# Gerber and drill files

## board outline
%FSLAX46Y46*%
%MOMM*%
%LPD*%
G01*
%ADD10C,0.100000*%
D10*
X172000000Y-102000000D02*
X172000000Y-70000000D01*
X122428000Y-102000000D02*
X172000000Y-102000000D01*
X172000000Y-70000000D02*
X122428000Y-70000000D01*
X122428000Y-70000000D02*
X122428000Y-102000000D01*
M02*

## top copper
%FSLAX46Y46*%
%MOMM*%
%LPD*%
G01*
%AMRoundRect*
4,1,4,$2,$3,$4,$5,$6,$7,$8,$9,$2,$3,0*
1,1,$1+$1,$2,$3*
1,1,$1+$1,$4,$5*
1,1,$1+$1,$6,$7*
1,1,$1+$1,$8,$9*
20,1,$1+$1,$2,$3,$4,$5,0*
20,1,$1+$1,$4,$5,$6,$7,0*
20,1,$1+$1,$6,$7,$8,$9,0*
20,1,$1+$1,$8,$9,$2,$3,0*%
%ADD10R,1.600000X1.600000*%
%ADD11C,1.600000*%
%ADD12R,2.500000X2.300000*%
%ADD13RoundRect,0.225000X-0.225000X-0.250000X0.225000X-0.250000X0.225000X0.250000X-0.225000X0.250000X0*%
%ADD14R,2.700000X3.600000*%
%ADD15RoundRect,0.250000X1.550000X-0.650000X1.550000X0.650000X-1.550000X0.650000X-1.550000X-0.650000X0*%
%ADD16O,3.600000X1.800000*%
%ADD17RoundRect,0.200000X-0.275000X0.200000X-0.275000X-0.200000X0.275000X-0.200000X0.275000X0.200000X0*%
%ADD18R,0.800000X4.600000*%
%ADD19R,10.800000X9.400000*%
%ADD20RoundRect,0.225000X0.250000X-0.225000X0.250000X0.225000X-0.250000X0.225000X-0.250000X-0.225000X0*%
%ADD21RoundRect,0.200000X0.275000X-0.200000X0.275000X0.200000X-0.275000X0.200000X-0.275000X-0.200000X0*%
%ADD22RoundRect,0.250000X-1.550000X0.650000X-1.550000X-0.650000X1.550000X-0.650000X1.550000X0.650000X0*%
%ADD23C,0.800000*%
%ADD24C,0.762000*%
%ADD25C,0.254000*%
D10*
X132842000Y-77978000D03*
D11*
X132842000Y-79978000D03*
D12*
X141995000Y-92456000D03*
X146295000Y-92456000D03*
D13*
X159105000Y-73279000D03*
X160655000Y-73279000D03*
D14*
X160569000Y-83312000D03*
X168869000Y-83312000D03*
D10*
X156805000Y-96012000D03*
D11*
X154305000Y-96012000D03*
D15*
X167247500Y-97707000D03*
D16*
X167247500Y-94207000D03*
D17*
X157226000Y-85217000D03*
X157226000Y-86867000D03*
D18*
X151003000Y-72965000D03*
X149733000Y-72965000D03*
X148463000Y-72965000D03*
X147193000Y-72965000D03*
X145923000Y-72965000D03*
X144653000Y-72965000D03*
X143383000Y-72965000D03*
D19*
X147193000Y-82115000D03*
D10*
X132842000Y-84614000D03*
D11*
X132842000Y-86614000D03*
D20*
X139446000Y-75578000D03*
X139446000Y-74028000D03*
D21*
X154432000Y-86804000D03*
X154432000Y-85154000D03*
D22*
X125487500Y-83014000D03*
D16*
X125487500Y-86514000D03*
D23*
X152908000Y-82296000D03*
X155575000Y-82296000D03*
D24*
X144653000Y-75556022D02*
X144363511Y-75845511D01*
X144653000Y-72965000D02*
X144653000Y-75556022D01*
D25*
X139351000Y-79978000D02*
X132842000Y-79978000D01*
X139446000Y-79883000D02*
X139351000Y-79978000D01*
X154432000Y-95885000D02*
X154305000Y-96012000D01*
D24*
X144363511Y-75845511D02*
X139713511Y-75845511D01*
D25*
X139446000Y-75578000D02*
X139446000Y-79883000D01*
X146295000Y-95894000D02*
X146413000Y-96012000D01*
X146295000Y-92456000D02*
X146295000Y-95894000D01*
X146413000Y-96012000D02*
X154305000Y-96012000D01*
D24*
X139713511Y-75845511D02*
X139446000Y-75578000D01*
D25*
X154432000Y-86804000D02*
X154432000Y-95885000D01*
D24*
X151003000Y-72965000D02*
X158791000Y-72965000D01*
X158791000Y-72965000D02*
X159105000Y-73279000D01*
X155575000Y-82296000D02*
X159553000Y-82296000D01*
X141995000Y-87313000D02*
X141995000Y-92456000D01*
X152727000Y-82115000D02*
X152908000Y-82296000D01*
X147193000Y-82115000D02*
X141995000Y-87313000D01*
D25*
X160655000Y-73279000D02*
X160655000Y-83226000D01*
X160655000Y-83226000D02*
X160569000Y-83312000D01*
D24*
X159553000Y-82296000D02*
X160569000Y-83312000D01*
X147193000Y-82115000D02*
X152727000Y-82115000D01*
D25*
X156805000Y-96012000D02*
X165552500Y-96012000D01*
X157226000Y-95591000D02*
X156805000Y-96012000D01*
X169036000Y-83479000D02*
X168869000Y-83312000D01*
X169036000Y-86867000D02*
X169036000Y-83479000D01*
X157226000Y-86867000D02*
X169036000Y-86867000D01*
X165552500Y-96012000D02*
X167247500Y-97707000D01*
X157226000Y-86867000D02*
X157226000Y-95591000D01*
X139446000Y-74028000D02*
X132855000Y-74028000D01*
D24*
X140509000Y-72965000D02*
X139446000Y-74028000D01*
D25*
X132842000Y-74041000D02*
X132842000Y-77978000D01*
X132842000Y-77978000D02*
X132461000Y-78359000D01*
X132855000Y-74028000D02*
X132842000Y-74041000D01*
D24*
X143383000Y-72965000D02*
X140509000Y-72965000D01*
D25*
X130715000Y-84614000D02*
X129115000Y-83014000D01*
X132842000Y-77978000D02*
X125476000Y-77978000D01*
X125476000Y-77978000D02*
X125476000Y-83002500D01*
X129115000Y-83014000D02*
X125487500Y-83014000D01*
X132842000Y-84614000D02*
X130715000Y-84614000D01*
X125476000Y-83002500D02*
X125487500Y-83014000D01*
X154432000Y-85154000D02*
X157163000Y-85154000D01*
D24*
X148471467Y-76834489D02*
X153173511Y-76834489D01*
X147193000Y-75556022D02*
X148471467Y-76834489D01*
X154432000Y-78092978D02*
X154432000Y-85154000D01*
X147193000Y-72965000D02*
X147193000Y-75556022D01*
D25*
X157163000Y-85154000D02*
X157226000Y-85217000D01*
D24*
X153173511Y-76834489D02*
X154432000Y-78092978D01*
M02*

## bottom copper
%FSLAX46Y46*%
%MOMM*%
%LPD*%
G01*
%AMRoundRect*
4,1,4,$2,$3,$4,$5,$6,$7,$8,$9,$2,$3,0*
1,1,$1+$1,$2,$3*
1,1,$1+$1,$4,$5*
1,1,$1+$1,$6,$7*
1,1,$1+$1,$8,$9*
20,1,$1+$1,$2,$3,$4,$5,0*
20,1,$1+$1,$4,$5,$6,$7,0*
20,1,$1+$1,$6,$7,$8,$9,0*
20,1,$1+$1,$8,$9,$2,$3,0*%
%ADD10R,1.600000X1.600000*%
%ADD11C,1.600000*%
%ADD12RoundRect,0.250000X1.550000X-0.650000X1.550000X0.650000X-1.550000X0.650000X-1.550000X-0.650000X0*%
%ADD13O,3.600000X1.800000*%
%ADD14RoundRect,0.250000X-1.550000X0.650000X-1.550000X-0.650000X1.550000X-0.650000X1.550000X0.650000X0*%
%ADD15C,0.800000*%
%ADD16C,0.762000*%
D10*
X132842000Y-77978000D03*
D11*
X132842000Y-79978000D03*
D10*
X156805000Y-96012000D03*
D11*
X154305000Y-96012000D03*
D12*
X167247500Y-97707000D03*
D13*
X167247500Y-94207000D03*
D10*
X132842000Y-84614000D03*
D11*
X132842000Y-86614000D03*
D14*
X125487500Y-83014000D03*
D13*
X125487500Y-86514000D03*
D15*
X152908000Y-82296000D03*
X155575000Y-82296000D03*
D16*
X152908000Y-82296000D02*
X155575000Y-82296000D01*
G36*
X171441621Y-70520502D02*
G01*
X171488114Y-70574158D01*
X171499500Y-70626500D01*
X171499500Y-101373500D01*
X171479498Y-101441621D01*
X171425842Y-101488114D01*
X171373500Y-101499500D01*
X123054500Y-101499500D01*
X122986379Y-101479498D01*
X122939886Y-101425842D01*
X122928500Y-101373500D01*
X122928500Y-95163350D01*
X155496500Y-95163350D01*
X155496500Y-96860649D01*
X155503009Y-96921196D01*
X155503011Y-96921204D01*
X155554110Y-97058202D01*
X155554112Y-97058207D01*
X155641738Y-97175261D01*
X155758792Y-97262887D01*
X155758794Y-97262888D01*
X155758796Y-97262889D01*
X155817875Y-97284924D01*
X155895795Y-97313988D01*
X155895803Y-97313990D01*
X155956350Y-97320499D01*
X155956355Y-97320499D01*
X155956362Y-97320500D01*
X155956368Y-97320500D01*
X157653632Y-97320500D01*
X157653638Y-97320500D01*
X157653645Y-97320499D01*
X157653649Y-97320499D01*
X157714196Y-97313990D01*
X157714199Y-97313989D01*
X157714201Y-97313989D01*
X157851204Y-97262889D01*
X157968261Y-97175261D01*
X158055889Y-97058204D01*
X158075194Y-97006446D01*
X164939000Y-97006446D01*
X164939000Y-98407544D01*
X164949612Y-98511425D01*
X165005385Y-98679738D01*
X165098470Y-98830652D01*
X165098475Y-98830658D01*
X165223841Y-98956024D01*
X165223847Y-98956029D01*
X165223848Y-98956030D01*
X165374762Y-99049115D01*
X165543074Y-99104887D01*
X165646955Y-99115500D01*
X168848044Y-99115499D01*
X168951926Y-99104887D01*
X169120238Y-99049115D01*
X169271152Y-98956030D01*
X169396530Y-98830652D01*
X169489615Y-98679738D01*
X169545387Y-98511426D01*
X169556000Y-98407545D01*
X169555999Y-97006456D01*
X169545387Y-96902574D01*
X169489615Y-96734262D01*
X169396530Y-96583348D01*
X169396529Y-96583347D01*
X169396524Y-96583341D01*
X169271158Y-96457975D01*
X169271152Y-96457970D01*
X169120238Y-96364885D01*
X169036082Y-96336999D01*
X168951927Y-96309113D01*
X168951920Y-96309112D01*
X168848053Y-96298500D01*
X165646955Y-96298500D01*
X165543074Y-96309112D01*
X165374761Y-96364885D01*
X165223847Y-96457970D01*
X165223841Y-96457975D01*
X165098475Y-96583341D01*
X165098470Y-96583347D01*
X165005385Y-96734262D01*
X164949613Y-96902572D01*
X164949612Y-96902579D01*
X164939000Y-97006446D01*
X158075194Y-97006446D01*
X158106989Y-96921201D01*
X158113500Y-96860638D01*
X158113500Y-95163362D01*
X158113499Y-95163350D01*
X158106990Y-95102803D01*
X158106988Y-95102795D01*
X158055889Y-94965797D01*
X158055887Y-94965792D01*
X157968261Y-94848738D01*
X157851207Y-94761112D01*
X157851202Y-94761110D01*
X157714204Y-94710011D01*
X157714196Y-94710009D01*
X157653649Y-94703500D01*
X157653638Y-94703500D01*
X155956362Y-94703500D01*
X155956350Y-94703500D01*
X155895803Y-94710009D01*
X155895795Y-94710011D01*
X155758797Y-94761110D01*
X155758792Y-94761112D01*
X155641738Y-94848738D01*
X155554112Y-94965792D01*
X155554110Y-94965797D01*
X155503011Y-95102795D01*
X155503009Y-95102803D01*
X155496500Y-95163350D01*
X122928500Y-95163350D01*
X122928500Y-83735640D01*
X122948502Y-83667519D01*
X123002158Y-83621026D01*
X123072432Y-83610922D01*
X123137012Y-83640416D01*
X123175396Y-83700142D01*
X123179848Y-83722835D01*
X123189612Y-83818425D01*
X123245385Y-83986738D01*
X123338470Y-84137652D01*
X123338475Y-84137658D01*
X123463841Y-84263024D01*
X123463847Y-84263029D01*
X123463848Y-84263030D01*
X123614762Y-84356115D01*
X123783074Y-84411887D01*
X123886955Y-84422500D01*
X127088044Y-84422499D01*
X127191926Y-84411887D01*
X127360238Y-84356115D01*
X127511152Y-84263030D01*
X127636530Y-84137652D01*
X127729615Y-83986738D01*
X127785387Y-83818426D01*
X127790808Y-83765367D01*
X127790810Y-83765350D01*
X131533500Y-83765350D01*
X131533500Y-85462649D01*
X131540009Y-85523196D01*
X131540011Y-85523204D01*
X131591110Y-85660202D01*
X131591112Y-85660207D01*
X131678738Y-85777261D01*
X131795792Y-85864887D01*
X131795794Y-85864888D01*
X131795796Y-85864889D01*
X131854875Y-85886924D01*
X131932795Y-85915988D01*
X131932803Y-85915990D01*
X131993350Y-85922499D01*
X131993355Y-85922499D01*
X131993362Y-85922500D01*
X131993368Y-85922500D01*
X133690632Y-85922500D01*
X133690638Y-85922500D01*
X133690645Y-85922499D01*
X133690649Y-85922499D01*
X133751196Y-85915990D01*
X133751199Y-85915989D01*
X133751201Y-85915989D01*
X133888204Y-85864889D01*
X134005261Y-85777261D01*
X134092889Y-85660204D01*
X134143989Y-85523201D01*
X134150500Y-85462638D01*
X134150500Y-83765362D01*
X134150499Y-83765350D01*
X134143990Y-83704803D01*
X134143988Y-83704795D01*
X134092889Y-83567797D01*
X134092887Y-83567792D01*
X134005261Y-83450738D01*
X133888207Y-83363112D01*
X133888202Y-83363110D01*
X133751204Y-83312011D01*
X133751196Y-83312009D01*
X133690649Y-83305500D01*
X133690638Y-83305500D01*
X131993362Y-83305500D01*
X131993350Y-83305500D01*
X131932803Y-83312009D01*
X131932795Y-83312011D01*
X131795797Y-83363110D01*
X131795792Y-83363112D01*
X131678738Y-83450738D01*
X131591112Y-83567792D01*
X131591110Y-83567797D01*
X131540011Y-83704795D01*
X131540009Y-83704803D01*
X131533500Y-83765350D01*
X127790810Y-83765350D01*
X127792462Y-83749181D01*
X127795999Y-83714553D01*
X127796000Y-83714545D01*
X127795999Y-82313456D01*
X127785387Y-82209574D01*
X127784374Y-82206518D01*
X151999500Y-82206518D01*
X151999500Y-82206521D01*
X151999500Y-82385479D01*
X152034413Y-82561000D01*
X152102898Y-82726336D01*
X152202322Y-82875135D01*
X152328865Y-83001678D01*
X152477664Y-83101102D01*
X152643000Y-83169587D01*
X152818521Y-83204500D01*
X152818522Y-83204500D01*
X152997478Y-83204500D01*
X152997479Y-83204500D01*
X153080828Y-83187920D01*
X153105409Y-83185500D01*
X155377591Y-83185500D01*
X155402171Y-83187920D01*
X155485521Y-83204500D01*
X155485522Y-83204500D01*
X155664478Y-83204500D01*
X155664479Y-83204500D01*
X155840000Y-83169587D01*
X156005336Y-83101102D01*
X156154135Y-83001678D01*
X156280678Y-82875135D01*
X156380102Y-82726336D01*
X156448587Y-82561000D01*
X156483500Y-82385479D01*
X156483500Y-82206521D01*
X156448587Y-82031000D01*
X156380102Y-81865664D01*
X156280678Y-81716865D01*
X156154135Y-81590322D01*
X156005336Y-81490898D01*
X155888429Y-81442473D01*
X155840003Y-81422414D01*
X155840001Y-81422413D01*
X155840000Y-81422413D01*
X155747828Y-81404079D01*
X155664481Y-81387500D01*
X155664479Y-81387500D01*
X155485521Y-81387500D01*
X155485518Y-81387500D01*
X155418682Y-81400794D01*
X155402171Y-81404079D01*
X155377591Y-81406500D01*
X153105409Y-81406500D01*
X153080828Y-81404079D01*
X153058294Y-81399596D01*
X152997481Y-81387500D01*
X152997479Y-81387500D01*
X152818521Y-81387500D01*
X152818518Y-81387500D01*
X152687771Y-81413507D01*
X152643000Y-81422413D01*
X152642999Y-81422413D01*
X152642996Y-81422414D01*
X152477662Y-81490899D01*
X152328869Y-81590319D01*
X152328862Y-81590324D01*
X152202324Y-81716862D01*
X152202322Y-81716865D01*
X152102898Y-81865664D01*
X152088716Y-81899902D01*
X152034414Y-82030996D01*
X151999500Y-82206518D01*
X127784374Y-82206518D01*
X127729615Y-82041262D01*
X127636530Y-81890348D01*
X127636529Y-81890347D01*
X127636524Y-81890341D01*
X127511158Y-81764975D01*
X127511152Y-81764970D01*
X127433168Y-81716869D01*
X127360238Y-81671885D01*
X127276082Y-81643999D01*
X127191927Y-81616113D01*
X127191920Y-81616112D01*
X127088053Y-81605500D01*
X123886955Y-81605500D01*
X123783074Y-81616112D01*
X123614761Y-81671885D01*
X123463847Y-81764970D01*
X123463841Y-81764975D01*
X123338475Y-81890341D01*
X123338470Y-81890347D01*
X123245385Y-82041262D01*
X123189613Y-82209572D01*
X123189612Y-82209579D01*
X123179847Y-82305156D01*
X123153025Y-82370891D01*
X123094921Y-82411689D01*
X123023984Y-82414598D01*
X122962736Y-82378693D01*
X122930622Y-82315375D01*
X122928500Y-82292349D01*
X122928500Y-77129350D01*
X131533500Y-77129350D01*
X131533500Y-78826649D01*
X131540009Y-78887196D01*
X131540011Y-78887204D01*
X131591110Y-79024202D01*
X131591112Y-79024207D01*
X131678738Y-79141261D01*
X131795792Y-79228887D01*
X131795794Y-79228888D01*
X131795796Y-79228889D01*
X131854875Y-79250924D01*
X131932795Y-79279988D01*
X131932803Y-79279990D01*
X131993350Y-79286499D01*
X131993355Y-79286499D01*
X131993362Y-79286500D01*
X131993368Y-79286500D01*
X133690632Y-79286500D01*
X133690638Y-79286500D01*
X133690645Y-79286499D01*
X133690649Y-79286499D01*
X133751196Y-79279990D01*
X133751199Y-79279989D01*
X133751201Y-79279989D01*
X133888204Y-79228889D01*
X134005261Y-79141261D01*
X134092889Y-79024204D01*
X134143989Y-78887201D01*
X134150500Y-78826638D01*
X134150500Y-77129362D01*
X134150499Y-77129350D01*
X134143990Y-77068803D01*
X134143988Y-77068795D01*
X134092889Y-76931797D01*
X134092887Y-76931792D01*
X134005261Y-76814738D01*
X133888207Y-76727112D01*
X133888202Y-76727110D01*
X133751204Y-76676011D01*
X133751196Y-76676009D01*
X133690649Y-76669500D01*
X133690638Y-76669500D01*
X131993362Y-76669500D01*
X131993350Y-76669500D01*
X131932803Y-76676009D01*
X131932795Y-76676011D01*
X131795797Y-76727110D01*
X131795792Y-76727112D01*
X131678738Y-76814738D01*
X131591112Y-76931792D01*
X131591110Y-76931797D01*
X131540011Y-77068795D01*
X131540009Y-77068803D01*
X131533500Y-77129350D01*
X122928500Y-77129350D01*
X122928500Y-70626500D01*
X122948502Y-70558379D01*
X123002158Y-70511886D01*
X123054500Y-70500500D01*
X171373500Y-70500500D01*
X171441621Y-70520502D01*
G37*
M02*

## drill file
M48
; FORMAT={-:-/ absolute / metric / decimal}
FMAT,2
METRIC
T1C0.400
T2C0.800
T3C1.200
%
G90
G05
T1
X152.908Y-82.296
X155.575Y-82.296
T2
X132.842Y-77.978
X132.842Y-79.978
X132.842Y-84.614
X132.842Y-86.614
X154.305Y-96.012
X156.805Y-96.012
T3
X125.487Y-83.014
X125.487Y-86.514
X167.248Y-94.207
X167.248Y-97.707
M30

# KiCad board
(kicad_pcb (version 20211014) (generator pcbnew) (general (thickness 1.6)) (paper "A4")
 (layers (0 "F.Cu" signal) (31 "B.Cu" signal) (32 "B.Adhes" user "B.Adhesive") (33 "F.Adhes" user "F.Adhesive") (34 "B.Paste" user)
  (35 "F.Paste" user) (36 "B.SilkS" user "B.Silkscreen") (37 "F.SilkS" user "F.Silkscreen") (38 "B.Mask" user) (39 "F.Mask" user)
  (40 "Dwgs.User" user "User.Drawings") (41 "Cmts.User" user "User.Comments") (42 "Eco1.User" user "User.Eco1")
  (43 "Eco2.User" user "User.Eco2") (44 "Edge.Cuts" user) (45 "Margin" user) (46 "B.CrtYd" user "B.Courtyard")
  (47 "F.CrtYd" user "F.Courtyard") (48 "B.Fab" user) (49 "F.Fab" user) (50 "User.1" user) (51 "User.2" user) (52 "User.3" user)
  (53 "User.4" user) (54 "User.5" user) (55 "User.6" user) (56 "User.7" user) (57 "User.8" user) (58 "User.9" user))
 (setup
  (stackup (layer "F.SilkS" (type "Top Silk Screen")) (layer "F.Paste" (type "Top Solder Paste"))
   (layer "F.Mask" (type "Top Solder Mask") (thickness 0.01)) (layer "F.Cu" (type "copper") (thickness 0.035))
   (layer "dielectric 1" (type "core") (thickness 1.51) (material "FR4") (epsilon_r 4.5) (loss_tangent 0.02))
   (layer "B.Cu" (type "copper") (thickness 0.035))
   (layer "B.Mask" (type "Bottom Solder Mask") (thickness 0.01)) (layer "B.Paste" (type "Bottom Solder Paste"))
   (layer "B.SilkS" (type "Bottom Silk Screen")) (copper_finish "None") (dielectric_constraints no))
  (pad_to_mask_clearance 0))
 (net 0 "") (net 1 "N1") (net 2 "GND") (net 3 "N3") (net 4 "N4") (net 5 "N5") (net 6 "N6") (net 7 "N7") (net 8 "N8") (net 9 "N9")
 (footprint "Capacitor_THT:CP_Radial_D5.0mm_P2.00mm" (layer "F.Cu") (at 132.842 77.978 -90)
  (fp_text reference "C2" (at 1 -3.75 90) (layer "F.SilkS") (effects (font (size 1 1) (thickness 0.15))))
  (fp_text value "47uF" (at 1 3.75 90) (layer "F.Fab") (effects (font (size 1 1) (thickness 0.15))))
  (pad "1" thru_hole rect (at 0 0 270) (size 1.6 1.6) (drill 0.8) (layers *.Cu *.Mask) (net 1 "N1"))
  (pad "2" thru_hole circle (at 2 0 270) (size 1.6 1.6) (drill 0.8) (layers *.Cu *.Mask) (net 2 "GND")))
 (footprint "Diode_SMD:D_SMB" (layer "F.Cu") (at 144.145 92.456)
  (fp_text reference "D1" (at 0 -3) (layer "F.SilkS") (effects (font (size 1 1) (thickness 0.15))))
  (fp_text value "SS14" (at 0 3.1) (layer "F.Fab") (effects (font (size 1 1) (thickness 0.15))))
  (pad "1" smd rect (at -2.15 0) (size 2.5 2.3) (layers "F.Cu" "F.Paste" "F.Mask") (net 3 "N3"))
  (pad "2" smd rect (at 2.15 0) (size 2.5 2.3) (layers "F.Cu" "F.Paste" "F.Mask") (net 2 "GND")))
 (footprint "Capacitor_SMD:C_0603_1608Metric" (layer "F.Cu") (at 159.88 73.279)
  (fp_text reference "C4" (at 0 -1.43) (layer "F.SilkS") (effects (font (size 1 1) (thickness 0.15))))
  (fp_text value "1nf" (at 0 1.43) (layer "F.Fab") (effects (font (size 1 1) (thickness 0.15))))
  (pad "1" smd roundrect (at -0.775 0) (size 0.9 0.95) (layers "F.Cu" "F.Paste" "F.Mask") (roundrect_rratio 0.25) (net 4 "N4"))
  (pad "2" smd roundrect (at 0.775 0) (size 0.9 0.95) (layers "F.Cu" "F.Paste" "F.Mask") (roundrect_rratio 0.25) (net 3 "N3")))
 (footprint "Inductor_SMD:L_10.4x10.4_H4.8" (layer "F.Cu") (at 164.719 83.312)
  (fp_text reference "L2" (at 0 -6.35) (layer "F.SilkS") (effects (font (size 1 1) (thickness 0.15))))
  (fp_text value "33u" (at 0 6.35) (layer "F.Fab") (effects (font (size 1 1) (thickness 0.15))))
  (pad "1" smd rect (at -4.15 0) (size 2.7 3.6) (layers "F.Cu" "F.Paste" "F.Mask") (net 3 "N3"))
  (pad "2" smd rect (at 4.15 0) (size 2.7 3.6) (layers "F.Cu" "F.Paste" "F.Mask") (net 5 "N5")))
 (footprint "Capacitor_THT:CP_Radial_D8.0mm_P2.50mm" (layer "F.Cu") (at 156.805 96.012 180)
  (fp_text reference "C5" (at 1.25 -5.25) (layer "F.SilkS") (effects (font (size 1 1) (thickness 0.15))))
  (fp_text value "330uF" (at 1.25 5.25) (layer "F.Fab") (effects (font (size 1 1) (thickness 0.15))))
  (pad "1" thru_hole rect (at 0 0 180) (size 1.6 1.6) (drill 0.8) (layers *.Cu *.Mask) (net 5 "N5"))
  (pad "2" thru_hole circle (at 2.5 0 180) (size 1.6 1.6) (drill 0.8) (layers *.Cu *.Mask) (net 2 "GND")))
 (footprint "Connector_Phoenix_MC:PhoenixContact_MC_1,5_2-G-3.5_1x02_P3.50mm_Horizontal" (layer "F.Cu") (at 167.2475 97.707 90)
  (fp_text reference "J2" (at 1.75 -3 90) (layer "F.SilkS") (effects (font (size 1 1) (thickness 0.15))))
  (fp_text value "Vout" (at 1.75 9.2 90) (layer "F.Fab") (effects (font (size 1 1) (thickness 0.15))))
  (pad "1" thru_hole roundrect (at 0 0 90) (size 1.8 3.6) (drill 1.2) (layers *.Cu *.Mask) (roundrect_rratio 0.1388888889) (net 5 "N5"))
  (pad "2" thru_hole oval (at 3.5 0 90) (size 1.8 3.6) (drill 1.2) (layers *.Cu *.Mask) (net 2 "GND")))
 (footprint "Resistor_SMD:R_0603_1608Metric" (layer "F.Cu") (at 157.226 86.042 -90)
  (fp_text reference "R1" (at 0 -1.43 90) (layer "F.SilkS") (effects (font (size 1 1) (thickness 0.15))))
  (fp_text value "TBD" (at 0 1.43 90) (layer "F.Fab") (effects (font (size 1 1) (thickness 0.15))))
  (pad "1" smd roundrect (at -0.825 0 270) (size 0.8 0.95) (layers "F.Cu" "F.Paste" "F.Mask") (roundrect_rratio 0.25) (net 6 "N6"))
  (pad "2" smd roundrect (at 0.825 0 270) (size 0.8 0.95) (layers "F.Cu" "F.Paste" "F.Mask") (roundrect_rratio 0.25) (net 5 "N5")))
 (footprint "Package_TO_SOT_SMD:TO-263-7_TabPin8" (layer "F.Cu") (at 147.193 78.74 -90)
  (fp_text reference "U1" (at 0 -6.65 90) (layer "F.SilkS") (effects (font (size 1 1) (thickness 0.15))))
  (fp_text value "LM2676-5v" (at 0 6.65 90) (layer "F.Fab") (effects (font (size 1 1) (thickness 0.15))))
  (pad "" smd rect (at 0.95 2.775 270) (size 4.55 5.25) (layers "F.Paste"))
  (pad "" smd rect (at 5.8 -2.775 270) (size 4.55 5.25) (layers "F.Paste"))
  (pad "" smd rect (at 5.8 2.775 270) (size 4.55 5.25) (layers "F.Paste"))
  (pad "" smd rect (at 0.95 -2.775 270) (size 4.55 5.25) (layers "F.Paste"))
  (pad "1" smd rect (at -5.775 -3.81 270) (size 4.6 0.8) (layers "F.Cu" "F.Paste" "F.Mask") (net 4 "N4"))
  (pad "2" smd rect (at -5.775 -2.54 270) (size 4.6 0.8) (layers "F.Cu" "F.Paste" "F.Mask") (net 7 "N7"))
  (pad "3" smd rect (at -5.775 -1.27 270) (size 4.6 0.8) (layers "F.Cu" "F.Paste" "F.Mask") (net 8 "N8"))
  (pad "4" smd rect (at -5.775 0 270) (size 4.6 0.8) (layers "F.Cu" "F.Paste" "F.Mask") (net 6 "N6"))
  (pad "5" smd rect (at -5.775 1.27 270) (size 4.6 0.8) (layers "F.Cu" "F.Paste" "F.Mask") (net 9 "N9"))
  (pad "6" smd rect (at -5.775 2.54 270) (size 4.6 0.8) (layers "F.Cu" "F.Paste" "F.Mask") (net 2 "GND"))
  (pad "7" smd rect (at -5.775 3.81 270) (size 4.6 0.8) (layers "F.Cu" "F.Paste" "F.Mask") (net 1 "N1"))
  (pad "8" smd rect (at 3.375 0 270) (size 9.4 10.8) (layers "F.Cu" "F.Mask") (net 3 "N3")))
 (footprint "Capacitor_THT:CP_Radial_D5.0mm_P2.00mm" (layer "F.Cu") (at 132.842 84.614 -90)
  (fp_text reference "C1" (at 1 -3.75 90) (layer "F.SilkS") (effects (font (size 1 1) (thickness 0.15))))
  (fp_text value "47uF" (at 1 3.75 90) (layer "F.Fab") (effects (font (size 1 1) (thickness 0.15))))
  (pad "1" thru_hole rect (at 0 0 270) (size 1.6 1.6) (drill 0.8) (layers *.Cu *.Mask) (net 1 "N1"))
  (pad "2" thru_hole circle (at 2 0 270) (size 1.6 1.6) (drill 0.8) (layers *.Cu *.Mask) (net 2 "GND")))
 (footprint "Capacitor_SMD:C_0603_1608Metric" (layer "F.Cu") (at 139.446 74.803 90)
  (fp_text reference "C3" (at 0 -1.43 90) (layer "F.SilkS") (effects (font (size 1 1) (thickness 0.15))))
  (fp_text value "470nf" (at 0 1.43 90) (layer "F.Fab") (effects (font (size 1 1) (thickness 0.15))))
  (pad "1" smd roundrect (at -0.775 0 90) (size 0.9 0.95) (layers "F.Cu" "F.Paste" "F.Mask") (roundrect_rratio 0.25) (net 2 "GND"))
  (pad "2" smd roundrect (at 0.775 0 90) (size 0.9 0.95) (layers "F.Cu" "F.Paste" "F.Mask") (roundrect_rratio 0.25) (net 1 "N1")))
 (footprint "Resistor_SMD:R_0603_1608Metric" (layer "F.Cu") (at 154.432 85.979 90)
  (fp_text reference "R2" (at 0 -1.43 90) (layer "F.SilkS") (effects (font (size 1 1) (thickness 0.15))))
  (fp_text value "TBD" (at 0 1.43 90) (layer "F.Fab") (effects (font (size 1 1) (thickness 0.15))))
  (pad "1" smd roundrect (at -0.825 0 90) (size 0.8 0.95) (layers "F.Cu" "F.Paste" "F.Mask") (roundrect_rratio 0.25) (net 2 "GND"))
  (pad "2" smd roundrect (at 0.825 0 90) (size 0.8 0.95) (layers "F.Cu" "F.Paste" "F.Mask") (roundrect_rratio 0.25) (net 6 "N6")))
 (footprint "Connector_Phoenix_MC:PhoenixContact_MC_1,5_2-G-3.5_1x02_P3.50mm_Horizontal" (layer "F.Cu") (at 125.4875 83.014 -90)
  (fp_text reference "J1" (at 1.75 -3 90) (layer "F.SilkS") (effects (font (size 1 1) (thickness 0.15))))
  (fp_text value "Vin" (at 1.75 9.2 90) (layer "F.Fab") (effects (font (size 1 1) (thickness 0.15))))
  (pad "1" thru_hole roundrect (at 0 0 270) (size 1.8 3.6) (drill 1.2) (layers *.Cu *.Mask) (roundrect_rratio 0.1388888889) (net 1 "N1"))
  (pad "2" thru_hole oval (at 3.5 0 270) (size 1.8 3.6) (drill 1.2) (layers *.Cu *.Mask) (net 2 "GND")))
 (gr_line (start 172 102) (end 172 70) (layer "Edge.Cuts") (width 0.1))
 (gr_line (start 122.428 102) (end 172 102) (layer "Edge.Cuts") (width 0.1))
 (gr_line (start 172 70) (end 122.428 70) (layer "Edge.Cuts") (width 0.1))
 (gr_line (start 122.428 70) (end 122.428 102) (layer "Edge.Cuts") (width 0.1))
 (segment (start 144.653 75.556022) (end 144.363511 75.845511) (width 0.762) (layer "F.Cu") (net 2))
 (segment (start 144.653 72.965) (end 144.653 75.556022) (width 0.762) (layer "F.Cu") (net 2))
 (segment (start 139.351 79.978) (end 132.842 79.978) (width 0.254) (layer "F.Cu") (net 2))
 (segment (start 139.446 79.883) (end 139.351 79.978) (width 0.254) (layer "F.Cu") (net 2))
 (segment (start 154.432 95.885) (end 154.305 96.012) (width 0.254) (layer "F.Cu") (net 2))
 (segment (start 144.363511 75.845511) (end 139.713511 75.845511) (width 0.762) (layer "F.Cu") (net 2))
 (segment (start 139.446 75.578) (end 139.446 79.883) (width 0.254) (layer "F.Cu") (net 2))
 (segment (start 146.295 95.894) (end 146.413 96.012) (width 0.254) (layer "F.Cu") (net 2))
 (segment (start 146.295 92.456) (end 146.295 95.894) (width 0.254) (layer "F.Cu") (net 2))
 (segment (start 146.413 96.012) (end 154.305 96.012) (width 0.254) (layer "F.Cu") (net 2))
 (segment (start 139.713511 75.845511) (end 139.446 75.578) (width 0.762) (layer "F.Cu") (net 2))
 (segment (start 154.432 86.804) (end 154.432 95.885) (width 0.254) (layer "F.Cu") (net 2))
 (segment (start 151.003 72.965) (end 158.791 72.965) (width 0.762) (layer "F.Cu") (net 4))
 (segment (start 158.791 72.965) (end 159.105 73.279) (width 0.762) (layer "F.Cu") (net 4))
 (segment (start 155.575 82.296) (end 159.553 82.296) (width 0.762) (layer "F.Cu") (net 3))
 (segment (start 141.995 87.313) (end 141.995 92.456) (width 0.762) (layer "F.Cu") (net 3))
 (segment (start 152.727 82.115) (end 152.908 82.296) (width 0.762) (layer "F.Cu") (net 3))
 (segment (start 147.193 82.115) (end 141.995 87.313) (width 0.762) (layer "F.Cu") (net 3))
 (segment (start 160.655 73.279) (end 160.655 83.226) (width 0.254) (layer "F.Cu") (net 3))
 (segment (start 160.655 83.226) (end 160.569 83.312) (width 0.254) (layer "F.Cu") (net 3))
 (segment (start 159.553 82.296) (end 160.569 83.312) (width 0.762) (layer "F.Cu") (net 3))
 (segment (start 147.193 82.115) (end 152.727 82.115) (width 0.762) (layer "F.Cu") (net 3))
 (via (at 152.908 82.296) (size 0.8) (drill 0.4) (layers "F.Cu" "B.Cu") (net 3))
 (via (at 155.575 82.296) (size 0.8) (drill 0.4) (layers "F.Cu" "B.Cu") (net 3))
 (segment (start 152.908 82.296) (end 155.575 82.296) (width 0.762) (layer "B.Cu") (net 3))
 (segment (start 156.805 96.012) (end 165.5525 96.012) (width 0.254) (layer "F.Cu") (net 5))
 (segment (start 157.226 95.591) (end 156.805 96.012) (width 0.254) (layer "F.Cu") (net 5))
 (segment (start 169.036 83.479) (end 168.869 83.312) (width 0.254) (layer "F.Cu") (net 5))
 (segment (start 169.036 86.867) (end 169.036 83.479) (width 0.254) (layer "F.Cu") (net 5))
 (segment (start 157.226 86.867) (end 169.036 86.867) (width 0.254) (layer "F.Cu") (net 5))
 (segment (start 165.5525 96.012) (end 167.2475 97.707) (width 0.254) (layer "F.Cu") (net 5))
 (segment (start 157.226 86.867) (end 157.226 95.591) (width 0.254) (layer "F.Cu") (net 5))
 (segment (start 139.446 74.028) (end 132.855 74.028) (width 0.254) (layer "F.Cu") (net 1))
 (segment (start 140.509 72.965) (end 139.446 74.028) (width 0.762) (layer "F.Cu") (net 1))
 (segment (start 132.842 74.041) (end 132.842 77.978) (width 0.254) (layer "F.Cu") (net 1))
 (segment (start 132.842 77.978) (end 132.461 78.359) (width 0.254) (layer "F.Cu") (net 1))
 (segment (start 132.855 74.028) (end 132.842 74.041) (width 0.254) (layer "F.Cu") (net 1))
 (segment (start 143.383 72.965) (end 140.509 72.965) (width 0.762) (layer "F.Cu") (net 1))
 (segment (start 130.715 84.614) (end 129.115 83.014) (width 0.254) (layer "F.Cu") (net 1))
 (segment (start 132.842 77.978) (end 125.476 77.978) (width 0.254) (layer "F.Cu") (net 1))
 (segment (start 125.476 77.978) (end 125.476 83.0025) (width 0.254) (layer "F.Cu") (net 1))
 (segment (start 129.115 83.014) (end 125.4875 83.014) (width 0.254) (layer "F.Cu") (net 1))
 (segment (start 132.842 84.614) (end 130.715 84.614) (width 0.254) (layer "F.Cu") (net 1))
 (segment (start 125.476 83.0025) (end 125.4875 83.014) (width 0.254) (layer "F.Cu") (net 1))
 (segment (start 154.432 85.154) (end 157.163 85.154) (width 0.254) (layer "F.Cu") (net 6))
 (segment (start 148.471467 76.834489) (end 153.173511 76.834489) (width 0.762) (layer "F.Cu") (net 6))
 (segment (start 147.193 75.556022) (end 148.471467 76.834489) (width 0.762) (layer "F.Cu") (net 6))
 (segment (start 154.432 78.092978) (end 154.432 85.154) (width 0.762) (layer "F.Cu") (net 6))
 (segment (start 147.193 72.965) (end 147.193 75.556022) (width 0.762) (layer "F.Cu") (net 6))
 (segment (start 157.163 85.154) (end 157.226 85.217) (width 0.254) (layer "F.Cu") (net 6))
 (segment (start 153.173511 76.834489) (end 154.432 78.092978) (width 0.762) (layer "F.Cu") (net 6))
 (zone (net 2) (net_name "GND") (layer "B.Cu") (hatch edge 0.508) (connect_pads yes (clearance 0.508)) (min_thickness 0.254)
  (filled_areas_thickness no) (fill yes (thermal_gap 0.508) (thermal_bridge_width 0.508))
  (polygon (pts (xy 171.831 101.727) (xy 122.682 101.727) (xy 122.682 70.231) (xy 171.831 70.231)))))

